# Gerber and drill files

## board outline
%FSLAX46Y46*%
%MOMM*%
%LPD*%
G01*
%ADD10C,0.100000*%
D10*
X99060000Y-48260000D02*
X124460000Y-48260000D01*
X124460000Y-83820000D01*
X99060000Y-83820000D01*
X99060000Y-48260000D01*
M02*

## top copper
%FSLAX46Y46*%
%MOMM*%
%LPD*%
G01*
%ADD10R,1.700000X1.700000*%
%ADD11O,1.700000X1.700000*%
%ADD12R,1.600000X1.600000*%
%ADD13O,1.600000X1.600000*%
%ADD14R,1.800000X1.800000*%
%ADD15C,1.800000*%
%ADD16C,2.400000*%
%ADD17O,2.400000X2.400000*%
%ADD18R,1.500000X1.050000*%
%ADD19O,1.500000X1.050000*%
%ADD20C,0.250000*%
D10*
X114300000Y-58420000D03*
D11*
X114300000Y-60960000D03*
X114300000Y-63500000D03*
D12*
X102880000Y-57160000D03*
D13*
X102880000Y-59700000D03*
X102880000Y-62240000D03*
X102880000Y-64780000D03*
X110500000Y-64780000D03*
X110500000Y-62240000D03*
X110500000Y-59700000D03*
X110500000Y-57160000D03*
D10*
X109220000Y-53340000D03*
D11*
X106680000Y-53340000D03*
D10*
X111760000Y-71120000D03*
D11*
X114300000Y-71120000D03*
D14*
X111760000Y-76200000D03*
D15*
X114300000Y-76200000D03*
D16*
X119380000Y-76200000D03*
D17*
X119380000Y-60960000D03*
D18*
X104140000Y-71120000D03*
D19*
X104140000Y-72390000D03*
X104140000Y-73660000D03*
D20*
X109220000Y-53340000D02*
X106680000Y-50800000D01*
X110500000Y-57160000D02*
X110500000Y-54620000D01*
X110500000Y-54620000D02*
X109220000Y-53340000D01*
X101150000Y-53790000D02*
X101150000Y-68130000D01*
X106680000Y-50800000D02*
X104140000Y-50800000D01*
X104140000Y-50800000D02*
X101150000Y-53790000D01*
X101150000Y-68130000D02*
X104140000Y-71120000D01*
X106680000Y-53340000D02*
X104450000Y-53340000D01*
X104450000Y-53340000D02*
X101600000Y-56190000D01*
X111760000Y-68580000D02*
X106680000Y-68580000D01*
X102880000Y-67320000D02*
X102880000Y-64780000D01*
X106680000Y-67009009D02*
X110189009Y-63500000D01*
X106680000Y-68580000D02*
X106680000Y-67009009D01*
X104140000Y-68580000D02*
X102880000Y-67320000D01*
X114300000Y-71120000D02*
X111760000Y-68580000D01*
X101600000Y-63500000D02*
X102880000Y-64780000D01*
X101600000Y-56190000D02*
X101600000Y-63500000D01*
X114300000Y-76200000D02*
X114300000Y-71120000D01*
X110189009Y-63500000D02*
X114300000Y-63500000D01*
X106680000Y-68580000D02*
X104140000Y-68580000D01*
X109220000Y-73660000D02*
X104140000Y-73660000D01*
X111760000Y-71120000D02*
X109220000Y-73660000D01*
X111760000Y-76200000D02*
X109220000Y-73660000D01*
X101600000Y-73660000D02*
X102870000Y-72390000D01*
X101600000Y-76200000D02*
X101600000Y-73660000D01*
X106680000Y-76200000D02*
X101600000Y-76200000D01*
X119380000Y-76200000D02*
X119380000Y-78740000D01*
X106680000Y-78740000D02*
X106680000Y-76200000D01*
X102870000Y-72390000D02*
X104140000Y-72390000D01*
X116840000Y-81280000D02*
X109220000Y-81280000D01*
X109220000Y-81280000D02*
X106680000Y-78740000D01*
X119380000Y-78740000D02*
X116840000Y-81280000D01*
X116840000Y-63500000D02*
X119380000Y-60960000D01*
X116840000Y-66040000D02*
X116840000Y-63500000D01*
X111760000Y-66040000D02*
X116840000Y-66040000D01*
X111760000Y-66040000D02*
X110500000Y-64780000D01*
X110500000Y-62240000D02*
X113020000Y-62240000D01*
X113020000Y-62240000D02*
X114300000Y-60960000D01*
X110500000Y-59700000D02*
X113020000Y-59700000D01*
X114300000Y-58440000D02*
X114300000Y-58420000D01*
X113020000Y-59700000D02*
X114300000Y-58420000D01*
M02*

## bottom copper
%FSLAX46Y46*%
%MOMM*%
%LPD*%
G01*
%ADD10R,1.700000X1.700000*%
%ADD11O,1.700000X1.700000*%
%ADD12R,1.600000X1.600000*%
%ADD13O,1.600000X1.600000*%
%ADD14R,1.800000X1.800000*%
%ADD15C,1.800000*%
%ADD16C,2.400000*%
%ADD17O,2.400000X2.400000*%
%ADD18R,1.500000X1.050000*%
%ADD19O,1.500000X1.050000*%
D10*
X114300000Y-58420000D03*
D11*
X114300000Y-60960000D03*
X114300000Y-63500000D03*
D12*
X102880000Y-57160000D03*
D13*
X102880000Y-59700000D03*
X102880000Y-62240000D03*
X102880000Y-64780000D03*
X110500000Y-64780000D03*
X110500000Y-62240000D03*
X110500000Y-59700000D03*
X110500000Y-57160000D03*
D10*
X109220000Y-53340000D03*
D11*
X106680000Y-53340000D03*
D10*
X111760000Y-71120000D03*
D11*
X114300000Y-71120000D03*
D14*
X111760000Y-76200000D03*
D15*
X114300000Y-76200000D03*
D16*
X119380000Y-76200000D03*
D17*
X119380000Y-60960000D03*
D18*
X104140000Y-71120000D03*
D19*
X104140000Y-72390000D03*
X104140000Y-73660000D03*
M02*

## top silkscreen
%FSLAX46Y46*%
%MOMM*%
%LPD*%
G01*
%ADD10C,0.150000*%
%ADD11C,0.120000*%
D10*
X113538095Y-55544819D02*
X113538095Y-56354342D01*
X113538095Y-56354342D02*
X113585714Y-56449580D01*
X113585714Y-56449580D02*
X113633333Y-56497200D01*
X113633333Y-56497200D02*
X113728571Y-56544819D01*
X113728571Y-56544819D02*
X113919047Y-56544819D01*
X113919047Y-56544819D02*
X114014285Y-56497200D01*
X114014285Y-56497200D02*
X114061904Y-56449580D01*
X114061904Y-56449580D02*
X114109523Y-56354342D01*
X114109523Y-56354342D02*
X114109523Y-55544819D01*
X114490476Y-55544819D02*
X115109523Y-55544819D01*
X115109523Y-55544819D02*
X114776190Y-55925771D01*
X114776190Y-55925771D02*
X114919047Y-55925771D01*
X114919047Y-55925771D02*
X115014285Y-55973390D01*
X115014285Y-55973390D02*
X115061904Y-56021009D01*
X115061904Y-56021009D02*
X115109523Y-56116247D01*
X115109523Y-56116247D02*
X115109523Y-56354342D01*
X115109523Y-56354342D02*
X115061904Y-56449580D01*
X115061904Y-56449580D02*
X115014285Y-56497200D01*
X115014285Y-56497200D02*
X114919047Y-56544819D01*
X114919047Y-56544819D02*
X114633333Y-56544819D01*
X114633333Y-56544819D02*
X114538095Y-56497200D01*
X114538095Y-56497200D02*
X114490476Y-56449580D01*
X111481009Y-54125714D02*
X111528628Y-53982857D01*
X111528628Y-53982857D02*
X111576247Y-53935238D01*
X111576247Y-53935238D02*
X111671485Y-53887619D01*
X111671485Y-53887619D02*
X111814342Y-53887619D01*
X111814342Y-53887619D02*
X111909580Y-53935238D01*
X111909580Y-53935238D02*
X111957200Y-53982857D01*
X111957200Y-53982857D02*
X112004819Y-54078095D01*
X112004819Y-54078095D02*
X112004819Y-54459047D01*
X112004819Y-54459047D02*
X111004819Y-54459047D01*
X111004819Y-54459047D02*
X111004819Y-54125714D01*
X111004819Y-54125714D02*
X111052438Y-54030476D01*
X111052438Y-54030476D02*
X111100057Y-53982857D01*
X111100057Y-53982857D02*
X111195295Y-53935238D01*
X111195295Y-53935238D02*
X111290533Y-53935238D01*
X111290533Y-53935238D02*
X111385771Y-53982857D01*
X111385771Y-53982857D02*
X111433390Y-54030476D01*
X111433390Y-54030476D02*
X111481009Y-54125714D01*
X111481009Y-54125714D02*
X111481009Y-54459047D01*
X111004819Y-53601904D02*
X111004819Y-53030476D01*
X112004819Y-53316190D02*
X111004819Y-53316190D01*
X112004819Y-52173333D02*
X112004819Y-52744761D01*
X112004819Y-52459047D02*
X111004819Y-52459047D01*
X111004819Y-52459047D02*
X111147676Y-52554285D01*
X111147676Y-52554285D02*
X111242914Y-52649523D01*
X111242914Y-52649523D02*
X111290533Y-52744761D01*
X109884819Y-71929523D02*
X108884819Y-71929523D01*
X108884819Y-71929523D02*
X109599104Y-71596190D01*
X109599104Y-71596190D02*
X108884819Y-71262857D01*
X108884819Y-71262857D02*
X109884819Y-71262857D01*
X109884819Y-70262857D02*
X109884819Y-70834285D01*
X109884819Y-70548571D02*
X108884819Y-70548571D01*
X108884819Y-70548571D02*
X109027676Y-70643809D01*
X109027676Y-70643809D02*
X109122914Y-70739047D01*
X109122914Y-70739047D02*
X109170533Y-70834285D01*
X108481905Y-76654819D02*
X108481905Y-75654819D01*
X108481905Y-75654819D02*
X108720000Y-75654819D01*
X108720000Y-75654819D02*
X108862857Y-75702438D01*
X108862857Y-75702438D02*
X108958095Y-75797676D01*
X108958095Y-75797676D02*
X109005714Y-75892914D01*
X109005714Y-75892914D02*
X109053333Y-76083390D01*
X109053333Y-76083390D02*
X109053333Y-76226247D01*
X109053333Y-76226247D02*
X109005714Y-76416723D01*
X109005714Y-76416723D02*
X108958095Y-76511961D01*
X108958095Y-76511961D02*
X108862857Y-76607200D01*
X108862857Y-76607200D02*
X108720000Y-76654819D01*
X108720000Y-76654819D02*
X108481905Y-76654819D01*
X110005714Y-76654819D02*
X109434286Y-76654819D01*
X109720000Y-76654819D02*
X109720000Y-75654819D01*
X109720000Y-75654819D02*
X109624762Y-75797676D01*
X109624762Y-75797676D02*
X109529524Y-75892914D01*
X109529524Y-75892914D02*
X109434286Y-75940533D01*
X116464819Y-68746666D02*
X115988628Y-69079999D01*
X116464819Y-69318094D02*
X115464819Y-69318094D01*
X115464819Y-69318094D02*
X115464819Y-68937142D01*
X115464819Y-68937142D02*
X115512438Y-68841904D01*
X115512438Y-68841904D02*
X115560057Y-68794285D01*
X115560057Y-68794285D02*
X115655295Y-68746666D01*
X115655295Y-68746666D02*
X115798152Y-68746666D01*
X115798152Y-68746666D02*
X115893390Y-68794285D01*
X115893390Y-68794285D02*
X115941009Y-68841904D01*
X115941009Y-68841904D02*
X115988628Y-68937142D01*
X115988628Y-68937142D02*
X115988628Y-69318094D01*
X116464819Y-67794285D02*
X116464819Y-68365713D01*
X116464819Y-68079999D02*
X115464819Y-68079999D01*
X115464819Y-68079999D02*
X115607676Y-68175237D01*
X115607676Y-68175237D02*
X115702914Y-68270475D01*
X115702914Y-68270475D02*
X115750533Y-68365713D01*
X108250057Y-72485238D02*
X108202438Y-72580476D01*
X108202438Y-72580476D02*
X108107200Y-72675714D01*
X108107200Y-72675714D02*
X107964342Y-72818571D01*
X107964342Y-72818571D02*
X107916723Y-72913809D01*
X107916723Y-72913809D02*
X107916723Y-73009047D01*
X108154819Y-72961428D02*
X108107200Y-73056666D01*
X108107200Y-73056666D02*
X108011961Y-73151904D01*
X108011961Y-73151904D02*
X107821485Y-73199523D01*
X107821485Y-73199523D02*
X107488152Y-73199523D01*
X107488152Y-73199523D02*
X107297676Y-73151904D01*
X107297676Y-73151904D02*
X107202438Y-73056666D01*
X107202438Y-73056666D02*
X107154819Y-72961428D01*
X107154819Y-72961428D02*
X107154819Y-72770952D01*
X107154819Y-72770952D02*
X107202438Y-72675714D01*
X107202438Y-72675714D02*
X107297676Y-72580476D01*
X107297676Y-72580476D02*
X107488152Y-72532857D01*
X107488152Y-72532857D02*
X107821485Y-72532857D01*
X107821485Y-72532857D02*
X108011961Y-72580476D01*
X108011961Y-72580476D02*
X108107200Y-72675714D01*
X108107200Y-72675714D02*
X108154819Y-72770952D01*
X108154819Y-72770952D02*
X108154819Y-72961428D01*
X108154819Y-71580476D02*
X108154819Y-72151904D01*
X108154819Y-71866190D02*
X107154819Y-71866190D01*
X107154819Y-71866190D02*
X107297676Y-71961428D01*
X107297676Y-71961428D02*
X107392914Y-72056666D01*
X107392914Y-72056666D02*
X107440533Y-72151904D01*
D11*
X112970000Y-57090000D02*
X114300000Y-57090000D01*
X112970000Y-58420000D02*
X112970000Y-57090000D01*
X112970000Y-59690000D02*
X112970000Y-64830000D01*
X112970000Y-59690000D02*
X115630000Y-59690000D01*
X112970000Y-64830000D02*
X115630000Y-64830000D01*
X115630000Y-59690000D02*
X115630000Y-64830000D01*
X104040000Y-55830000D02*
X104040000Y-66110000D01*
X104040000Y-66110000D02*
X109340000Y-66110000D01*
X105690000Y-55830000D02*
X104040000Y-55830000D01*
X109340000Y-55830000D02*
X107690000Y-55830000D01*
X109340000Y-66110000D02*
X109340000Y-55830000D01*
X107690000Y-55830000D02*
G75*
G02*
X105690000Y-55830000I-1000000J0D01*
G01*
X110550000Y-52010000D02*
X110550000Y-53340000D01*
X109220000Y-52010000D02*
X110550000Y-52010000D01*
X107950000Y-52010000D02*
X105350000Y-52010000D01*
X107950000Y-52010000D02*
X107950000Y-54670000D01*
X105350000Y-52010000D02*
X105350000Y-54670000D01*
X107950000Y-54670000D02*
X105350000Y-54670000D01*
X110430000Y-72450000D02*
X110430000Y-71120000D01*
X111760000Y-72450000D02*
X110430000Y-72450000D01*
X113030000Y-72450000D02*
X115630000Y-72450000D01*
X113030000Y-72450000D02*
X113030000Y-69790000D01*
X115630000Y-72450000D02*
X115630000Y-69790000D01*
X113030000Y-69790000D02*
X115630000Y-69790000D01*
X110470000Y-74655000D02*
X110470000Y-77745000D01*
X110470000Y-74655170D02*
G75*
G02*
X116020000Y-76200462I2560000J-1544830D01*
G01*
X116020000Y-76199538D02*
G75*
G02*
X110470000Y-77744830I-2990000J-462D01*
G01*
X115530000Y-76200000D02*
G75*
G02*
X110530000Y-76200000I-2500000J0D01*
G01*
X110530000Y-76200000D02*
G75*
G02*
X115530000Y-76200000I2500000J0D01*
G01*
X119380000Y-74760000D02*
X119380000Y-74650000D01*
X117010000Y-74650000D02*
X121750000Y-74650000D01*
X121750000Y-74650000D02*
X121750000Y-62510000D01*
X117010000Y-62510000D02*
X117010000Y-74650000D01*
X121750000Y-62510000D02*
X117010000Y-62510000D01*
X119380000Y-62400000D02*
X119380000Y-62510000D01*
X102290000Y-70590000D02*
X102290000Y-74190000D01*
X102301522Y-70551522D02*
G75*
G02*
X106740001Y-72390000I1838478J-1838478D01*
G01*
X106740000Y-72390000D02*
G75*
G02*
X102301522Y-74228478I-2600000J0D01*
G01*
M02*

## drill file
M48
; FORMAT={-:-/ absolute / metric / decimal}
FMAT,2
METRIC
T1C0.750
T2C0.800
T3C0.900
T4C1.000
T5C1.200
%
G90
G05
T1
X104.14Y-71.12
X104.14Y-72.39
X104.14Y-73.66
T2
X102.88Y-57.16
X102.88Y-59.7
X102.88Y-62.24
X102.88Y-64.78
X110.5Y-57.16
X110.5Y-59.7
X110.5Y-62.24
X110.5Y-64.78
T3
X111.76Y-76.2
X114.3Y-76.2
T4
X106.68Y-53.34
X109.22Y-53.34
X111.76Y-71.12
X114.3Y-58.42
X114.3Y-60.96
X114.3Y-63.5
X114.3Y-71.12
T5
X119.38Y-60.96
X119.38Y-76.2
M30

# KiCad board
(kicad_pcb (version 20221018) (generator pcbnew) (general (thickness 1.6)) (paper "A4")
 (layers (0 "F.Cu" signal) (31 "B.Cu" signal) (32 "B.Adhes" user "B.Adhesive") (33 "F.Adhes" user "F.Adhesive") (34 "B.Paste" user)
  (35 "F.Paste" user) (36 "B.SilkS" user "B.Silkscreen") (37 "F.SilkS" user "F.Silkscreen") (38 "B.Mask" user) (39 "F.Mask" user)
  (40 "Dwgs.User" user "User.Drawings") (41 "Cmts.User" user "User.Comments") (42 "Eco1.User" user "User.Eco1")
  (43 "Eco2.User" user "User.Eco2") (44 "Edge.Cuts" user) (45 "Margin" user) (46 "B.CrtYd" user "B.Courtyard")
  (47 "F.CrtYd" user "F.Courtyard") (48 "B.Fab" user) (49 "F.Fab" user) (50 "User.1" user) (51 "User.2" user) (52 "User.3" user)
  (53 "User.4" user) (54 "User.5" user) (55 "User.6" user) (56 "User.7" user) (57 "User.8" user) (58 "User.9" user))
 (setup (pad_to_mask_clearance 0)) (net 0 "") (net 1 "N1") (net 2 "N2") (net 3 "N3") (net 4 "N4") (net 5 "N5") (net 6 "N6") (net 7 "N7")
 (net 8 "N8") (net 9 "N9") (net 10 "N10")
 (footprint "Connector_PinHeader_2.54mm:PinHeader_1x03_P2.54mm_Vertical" (layer "F.Cu") (at 114.3 58.42)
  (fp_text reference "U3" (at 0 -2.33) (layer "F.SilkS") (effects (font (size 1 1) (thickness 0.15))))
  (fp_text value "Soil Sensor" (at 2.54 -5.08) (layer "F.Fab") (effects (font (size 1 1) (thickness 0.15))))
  (fp_line (start -1.33 -1.33) (end 0 -1.33) (stroke (width 0.12) (type solid)) (layer "F.SilkS"))
  (fp_line (start -1.33 0) (end -1.33 -1.33) (stroke (width 0.12) (type solid)) (layer "F.SilkS"))
  (fp_line (start -1.33 1.27) (end -1.33 6.41) (stroke (width 0.12) (type solid)) (layer "F.SilkS"))
  (fp_line (start -1.33 1.27) (end 1.33 1.27) (stroke (width 0.12) (type solid)) (layer "F.SilkS"))
  (fp_line (start -1.33 6.41) (end 1.33 6.41) (stroke (width 0.12) (type solid)) (layer "F.SilkS"))
  (fp_line (start 1.33 1.27) (end 1.33 6.41) (stroke (width 0.12) (type solid)) (layer "F.SilkS"))
  (pad "1" thru_hole rect (at 0 0) (size 1.7 1.7) (drill 1) (layers "*.Cu" "*.Mask") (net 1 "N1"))
  (pad "2" thru_hole oval (at 0 2.54) (size 1.7 1.7) (drill 1) (layers "*.Cu" "*.Mask") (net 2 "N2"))
  (pad "3" thru_hole oval (at 0 5.08) (size 1.7 1.7) (drill 1) (layers "*.Cu" "*.Mask") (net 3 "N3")))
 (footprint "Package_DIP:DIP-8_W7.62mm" (layer "F.Cu") (at 102.88 57.16)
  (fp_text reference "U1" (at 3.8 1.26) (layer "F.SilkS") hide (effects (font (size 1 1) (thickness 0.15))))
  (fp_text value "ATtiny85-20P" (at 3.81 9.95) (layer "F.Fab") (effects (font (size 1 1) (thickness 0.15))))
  (fp_line (start 1.16 -1.33) (end 1.16 8.95) (stroke (width 0.12) (type solid)) (layer "F.SilkS"))
  (fp_line (start 1.16 8.95) (end 6.46 8.95) (stroke (width 0.12) (type solid)) (layer "F.SilkS"))
  (fp_line (start 2.81 -1.33) (end 1.16 -1.33) (stroke (width 0.12) (type solid)) (layer "F.SilkS"))
  (fp_line (start 6.46 -1.33) (end 4.81 -1.33) (stroke (width 0.12) (type solid)) (layer "F.SilkS"))
  (fp_line (start 6.46 8.95) (end 6.46 -1.33) (stroke (width 0.12) (type solid)) (layer "F.SilkS"))
  (fp_arc (start 4.81 -1.33) (mid 3.81 -0.33) (end 2.81 -1.33) (stroke (width 0.12) (type solid)) (layer "F.SilkS"))
  (pad "1" thru_hole rect (at 0 0) (size 1.6 1.6) (drill 0.8) (layers "*.Cu" "*.Mask") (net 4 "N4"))
  (pad "2" thru_hole oval (at 0 2.54) (size 1.6 1.6) (drill 0.8) (layers "*.Cu" "*.Mask") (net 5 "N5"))
  (pad "3" thru_hole oval (at 0 5.08) (size 1.6 1.6) (drill 0.8) (layers "*.Cu" "*.Mask") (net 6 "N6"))
  (pad "4" thru_hole oval (at 0 7.62) (size 1.6 1.6) (drill 0.8) (layers "*.Cu" "*.Mask") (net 3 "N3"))
  (pad "5" thru_hole oval (at 7.62 7.62) (size 1.6 1.6) (drill 0.8) (layers "*.Cu" "*.Mask") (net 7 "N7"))
  (pad "6" thru_hole oval (at 7.62 5.08) (size 1.6 1.6) (drill 0.8) (layers "*.Cu" "*.Mask") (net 2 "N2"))
  (pad "7" thru_hole oval (at 7.62 2.54) (size 1.6 1.6) (drill 0.8) (layers "*.Cu" "*.Mask") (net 1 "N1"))
  (pad "8" thru_hole oval (at 7.62 0) (size 1.6 1.6) (drill 0.8) (layers "*.Cu" "*.Mask") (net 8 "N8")))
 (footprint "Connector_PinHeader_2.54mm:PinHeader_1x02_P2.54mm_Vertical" (layer "F.Cu") (at 109.22 53.34 -90)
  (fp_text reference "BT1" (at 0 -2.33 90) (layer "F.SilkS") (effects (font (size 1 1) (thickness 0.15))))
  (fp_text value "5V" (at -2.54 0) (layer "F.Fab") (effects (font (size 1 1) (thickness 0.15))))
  (fp_line (start -1.33 -1.33) (end 0 -1.33) (stroke (width 0.12) (type solid)) (layer "F.SilkS"))
  (fp_line (start -1.33 0) (end -1.33 -1.33) (stroke (width 0.12) (type solid)) (layer "F.SilkS"))
  (fp_line (start -1.33 1.27) (end -1.33 3.87) (stroke (width 0.12) (type solid)) (layer "F.SilkS"))
  (fp_line (start -1.33 1.27) (end 1.33 1.27) (stroke (width 0.12) (type solid)) (layer "F.SilkS"))
  (fp_line (start -1.33 3.87) (end 1.33 3.87) (stroke (width 0.12) (type solid)) (layer "F.SilkS"))
  (fp_line (start 1.33 1.27) (end 1.33 3.87) (stroke (width 0.12) (type solid)) (layer "F.SilkS"))
  (pad "1" thru_hole rect (at 0 0 270) (size 1.7 1.7) (drill 1) (layers "*.Cu" "*.Mask") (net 8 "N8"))
  (pad "2" thru_hole oval (at 0 2.54 270) (size 1.7 1.7) (drill 1) (layers "*.Cu" "*.Mask") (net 3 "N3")))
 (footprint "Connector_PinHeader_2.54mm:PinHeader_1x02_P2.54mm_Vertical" (layer "F.Cu") (at 111.76 71.12 90)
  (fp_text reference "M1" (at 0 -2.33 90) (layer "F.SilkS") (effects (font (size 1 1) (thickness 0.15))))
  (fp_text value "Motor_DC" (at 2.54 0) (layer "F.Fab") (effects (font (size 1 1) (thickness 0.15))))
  (fp_line (start -1.33 -1.33) (end 0 -1.33) (stroke (width 0.12) (type solid)) (layer "F.SilkS"))
  (fp_line (start -1.33 0) (end -1.33 -1.33) (stroke (width 0.12) (type solid)) (layer "F.SilkS"))
  (fp_line (start -1.33 1.27) (end -1.33 3.87) (stroke (width 0.12) (type solid)) (layer "F.SilkS"))
  (fp_line (start -1.33 1.27) (end 1.33 1.27) (stroke (width 0.12) (type solid)) (layer "F.SilkS"))
  (fp_line (start -1.33 3.87) (end 1.33 3.87) (stroke (width 0.12) (type solid)) (layer "F.SilkS"))
  (fp_line (start 1.33 1.27) (end 1.33 3.87) (stroke (width 0.12) (type solid)) (layer "F.SilkS"))
  (pad "1" thru_hole rect (at 0 0 90) (size 1.7 1.7) (drill 1) (layers "*.Cu" "*.Mask") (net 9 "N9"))
  (pad "2" thru_hole oval (at 0 2.54 90) (size 1.7 1.7) (drill 1) (layers "*.Cu" "*.Mask") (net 3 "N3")))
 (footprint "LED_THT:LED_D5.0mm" (layer "F.Cu") (at 111.76 76.2)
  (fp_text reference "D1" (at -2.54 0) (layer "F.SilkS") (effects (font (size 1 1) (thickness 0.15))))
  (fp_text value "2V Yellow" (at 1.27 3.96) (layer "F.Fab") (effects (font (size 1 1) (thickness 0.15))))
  (fp_line (start -1.29 -1.545) (end -1.29 1.545) (stroke (width 0.12) (type solid)) (layer "F.SilkS"))
  (fp_arc (start -1.29 -1.54483) (mid 2.072002 -2.880433) (end 4.26 0.000462) (stroke (width 0.12) (type solid)) (layer "F.SilkS"))
  (fp_arc (start 4.26 -0.000462) (mid 2.072002 2.880433) (end -1.29 1.54483) (stroke (width 0.12) (type solid)) (layer "F.SilkS"))
  (fp_circle (center 1.27 0) (end 3.77 0) (stroke (width 0.12) (type solid)) (fill none) (layer "F.SilkS"))
  (pad "1" thru_hole rect (at 0 0) (size 1.8 1.8) (drill 0.9) (layers "*.Cu" "*.Mask") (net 9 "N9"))
  (pad "2" thru_hole circle (at 2.54 0) (size 1.8 1.8) (drill 0.9) (layers "*.Cu" "*.Mask") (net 3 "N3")))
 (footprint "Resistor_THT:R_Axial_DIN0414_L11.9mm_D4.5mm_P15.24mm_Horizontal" (layer "F.Cu") (at 119.38 76.2 90)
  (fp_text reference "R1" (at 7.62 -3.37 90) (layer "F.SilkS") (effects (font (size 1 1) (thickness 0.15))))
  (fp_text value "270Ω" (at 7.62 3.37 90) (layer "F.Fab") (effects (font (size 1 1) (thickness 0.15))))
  (fp_line (start 1.44 0) (end 1.55 0) (stroke (width 0.12) (type solid)) (layer "F.SilkS"))
  (fp_line (start 1.55 -2.37) (end 1.55 2.37) (stroke (width 0.12) (type solid)) (layer "F.SilkS"))
  (fp_line (start 1.55 2.37) (end 13.69 2.37) (stroke (width 0.12) (type solid)) (layer "F.SilkS"))
  (fp_line (start 13.69 -2.37) (end 1.55 -2.37) (stroke (width 0.12) (type solid)) (layer "F.SilkS"))
  (fp_line (start 13.69 2.37) (end 13.69 -2.37) (stroke (width 0.12) (type solid)) (layer "F.SilkS"))
  (fp_line (start 13.8 0) (end 13.69 0) (stroke (width 0.12) (type solid)) (layer "F.SilkS"))
  (pad "1" thru_hole circle (at 0 0 90) (size 2.4 2.4) (drill 1.2) (layers "*.Cu" "*.Mask") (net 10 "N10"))
  (pad "2" thru_hole oval (at 15.24 0 90) (size 2.4 2.4) (drill 1.2) (layers "*.Cu" "*.Mask") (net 7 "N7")))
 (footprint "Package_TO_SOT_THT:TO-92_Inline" (layer "F.Cu") (at 104.14 71.12 -90)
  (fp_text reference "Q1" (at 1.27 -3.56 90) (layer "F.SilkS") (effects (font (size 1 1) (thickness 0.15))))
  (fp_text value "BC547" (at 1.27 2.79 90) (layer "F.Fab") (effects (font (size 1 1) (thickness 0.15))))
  (fp_line (start -0.53 1.85) (end 3.07 1.85) (stroke (width 0.12) (type solid)) (layer "F.SilkS"))
  (fp_arc (start -0.568478 1.838478) (mid -1.132087 -0.994977) (end 1.27 -2.6) (stroke (width 0.12) (type solid)) (layer "F.SilkS"))
  (fp_arc (start 1.27 -2.6) (mid 3.672087 -0.994977) (end 3.108478 1.838478) (stroke (width 0.12) (type solid)) (layer "F.SilkS"))
  (pad "1" thru_hole rect (at 0 0 270) (size 1.05 1.5) (drill 0.75) (layers "*.Cu" "*.Mask") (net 8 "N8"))
  (pad "2" thru_hole oval (at 1.27 0 270) (size 1.05 1.5) (drill 0.75) (layers "*.Cu" "*.Mask") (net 10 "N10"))
  (pad "3" thru_hole oval (at 2.54 0 270) (size 1.05 1.5) (drill 0.75) (layers "*.Cu" "*.Mask") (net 9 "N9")))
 (gr_rect (start 99.06 48.26) (end 124.46 83.82) (stroke (width 0.1) (type default)) (fill none) (layer "Edge.Cuts"))
 (segment (start 109.22 53.34) (end 106.68 50.8) (width 0.25) (layer "F.Cu") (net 8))
 (segment (start 110.5 57.16) (end 110.5 54.62) (width 0.25) (layer "F.Cu") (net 8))
 (segment (start 110.5 54.62) (end 109.22 53.34) (width 0.25) (layer "F.Cu") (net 8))
 (segment (start 101.15 53.79) (end 101.15 68.13) (width 0.25) (layer "F.Cu") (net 8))
 (segment (start 106.68 50.8) (end 104.14 50.8) (width 0.25) (layer "F.Cu") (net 8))
 (segment (start 104.14 50.8) (end 101.15 53.79) (width 0.25) (layer "F.Cu") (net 8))
 (segment (start 101.15 68.13) (end 104.14 71.12) (width 0.25) (layer "F.Cu") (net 8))
 (segment (start 106.68 53.34) (end 104.45 53.34) (width 0.25) (layer "F.Cu") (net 3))
 (segment (start 104.45 53.34) (end 101.6 56.19) (width 0.25) (layer "F.Cu") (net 3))
 (segment (start 111.76 68.58) (end 106.68 68.58) (width 0.25) (layer "F.Cu") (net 3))
 (segment (start 102.88 67.32) (end 102.88 64.78) (width 0.25) (layer "F.Cu") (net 3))
 (segment (start 106.68 67.009009) (end 110.189009 63.5) (width 0.25) (layer "F.Cu") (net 3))
 (segment (start 106.68 68.58) (end 106.68 67.009009) (width 0.25) (layer "F.Cu") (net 3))
 (segment (start 104.14 68.58) (end 102.88 67.32) (width 0.25) (layer "F.Cu") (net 3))
 (segment (start 114.3 71.12) (end 111.76 68.58) (width 0.25) (layer "F.Cu") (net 3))
 (segment (start 101.6 63.5) (end 102.88 64.78) (width 0.25) (layer "F.Cu") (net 3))
 (segment (start 101.6 56.19) (end 101.6 63.5) (width 0.25) (layer "F.Cu") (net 3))
 (segment (start 114.3 76.2) (end 114.3 71.12) (width 0.25) (layer "F.Cu") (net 3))
 (segment (start 110.189009 63.5) (end 114.3 63.5) (width 0.25) (layer "F.Cu") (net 3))
 (segment (start 106.68 68.58) (end 104.14 68.58) (width 0.25) (layer "F.Cu") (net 3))
 (segment (start 109.22 73.66) (end 104.14 73.66) (width 0.25) (layer "F.Cu") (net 9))
 (segment (start 111.76 71.12) (end 109.22 73.66) (width 0.25) (layer "F.Cu") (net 9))
 (segment (start 111.76 76.2) (end 109.22 73.66) (width 0.25) (layer "F.Cu") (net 9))
 (segment (start 101.6 73.66) (end 102.87 72.39) (width 0.25) (layer "F.Cu") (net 10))
 (segment (start 101.6 76.2) (end 101.6 73.66) (width 0.25) (layer "F.Cu") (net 10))
 (segment (start 106.68 76.2) (end 101.6 76.2) (width 0.25) (layer "F.Cu") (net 10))
 (segment (start 119.38 76.2) (end 119.38 78.74) (width 0.25) (layer "F.Cu") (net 10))
 (segment (start 106.68 78.74) (end 106.68 76.2) (width 0.25) (layer "F.Cu") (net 10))
 (segment (start 102.87 72.39) (end 104.14 72.39) (width 0.25) (layer "F.Cu") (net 10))
 (segment (start 116.84 81.28) (end 109.22 81.28) (width 0.25) (layer "F.Cu") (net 10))
 (segment (start 109.22 81.28) (end 106.68 78.74) (width 0.25) (layer "F.Cu") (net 10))
 (segment (start 119.38 78.74) (end 116.84 81.28) (width 0.25) (layer "F.Cu") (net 10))
 (segment (start 116.84 63.5) (end 119.38 60.96) (width 0.25) (layer "F.Cu") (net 7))
 (segment (start 116.84 66.04) (end 116.84 63.5) (width 0.25) (layer "F.Cu") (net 7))
 (segment (start 111.76 66.04) (end 116.84 66.04) (width 0.25) (layer "F.Cu") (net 7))
 (segment (start 111.76 66.04) (end 110.5 64.78) (width 0.25) (layer "F.Cu") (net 7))
 (segment (start 110.5 62.24) (end 113.02 62.24) (width 0.25) (layer "F.Cu") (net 2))
 (segment (start 113.02 62.24) (end 114.3 60.96) (width 0.25) (layer "F.Cu") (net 2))
 (segment (start 110.5 59.7) (end 113.02 59.7) (width 0.25) (layer "F.Cu") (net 1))
 (segment (start 114.3 58.44) (end 114.3 58.42) (width 0.25) (layer "F.Cu") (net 1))
 (segment (start 113.02 59.7) (end 114.3 58.42) (width 0.25) (layer "F.Cu") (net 1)))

